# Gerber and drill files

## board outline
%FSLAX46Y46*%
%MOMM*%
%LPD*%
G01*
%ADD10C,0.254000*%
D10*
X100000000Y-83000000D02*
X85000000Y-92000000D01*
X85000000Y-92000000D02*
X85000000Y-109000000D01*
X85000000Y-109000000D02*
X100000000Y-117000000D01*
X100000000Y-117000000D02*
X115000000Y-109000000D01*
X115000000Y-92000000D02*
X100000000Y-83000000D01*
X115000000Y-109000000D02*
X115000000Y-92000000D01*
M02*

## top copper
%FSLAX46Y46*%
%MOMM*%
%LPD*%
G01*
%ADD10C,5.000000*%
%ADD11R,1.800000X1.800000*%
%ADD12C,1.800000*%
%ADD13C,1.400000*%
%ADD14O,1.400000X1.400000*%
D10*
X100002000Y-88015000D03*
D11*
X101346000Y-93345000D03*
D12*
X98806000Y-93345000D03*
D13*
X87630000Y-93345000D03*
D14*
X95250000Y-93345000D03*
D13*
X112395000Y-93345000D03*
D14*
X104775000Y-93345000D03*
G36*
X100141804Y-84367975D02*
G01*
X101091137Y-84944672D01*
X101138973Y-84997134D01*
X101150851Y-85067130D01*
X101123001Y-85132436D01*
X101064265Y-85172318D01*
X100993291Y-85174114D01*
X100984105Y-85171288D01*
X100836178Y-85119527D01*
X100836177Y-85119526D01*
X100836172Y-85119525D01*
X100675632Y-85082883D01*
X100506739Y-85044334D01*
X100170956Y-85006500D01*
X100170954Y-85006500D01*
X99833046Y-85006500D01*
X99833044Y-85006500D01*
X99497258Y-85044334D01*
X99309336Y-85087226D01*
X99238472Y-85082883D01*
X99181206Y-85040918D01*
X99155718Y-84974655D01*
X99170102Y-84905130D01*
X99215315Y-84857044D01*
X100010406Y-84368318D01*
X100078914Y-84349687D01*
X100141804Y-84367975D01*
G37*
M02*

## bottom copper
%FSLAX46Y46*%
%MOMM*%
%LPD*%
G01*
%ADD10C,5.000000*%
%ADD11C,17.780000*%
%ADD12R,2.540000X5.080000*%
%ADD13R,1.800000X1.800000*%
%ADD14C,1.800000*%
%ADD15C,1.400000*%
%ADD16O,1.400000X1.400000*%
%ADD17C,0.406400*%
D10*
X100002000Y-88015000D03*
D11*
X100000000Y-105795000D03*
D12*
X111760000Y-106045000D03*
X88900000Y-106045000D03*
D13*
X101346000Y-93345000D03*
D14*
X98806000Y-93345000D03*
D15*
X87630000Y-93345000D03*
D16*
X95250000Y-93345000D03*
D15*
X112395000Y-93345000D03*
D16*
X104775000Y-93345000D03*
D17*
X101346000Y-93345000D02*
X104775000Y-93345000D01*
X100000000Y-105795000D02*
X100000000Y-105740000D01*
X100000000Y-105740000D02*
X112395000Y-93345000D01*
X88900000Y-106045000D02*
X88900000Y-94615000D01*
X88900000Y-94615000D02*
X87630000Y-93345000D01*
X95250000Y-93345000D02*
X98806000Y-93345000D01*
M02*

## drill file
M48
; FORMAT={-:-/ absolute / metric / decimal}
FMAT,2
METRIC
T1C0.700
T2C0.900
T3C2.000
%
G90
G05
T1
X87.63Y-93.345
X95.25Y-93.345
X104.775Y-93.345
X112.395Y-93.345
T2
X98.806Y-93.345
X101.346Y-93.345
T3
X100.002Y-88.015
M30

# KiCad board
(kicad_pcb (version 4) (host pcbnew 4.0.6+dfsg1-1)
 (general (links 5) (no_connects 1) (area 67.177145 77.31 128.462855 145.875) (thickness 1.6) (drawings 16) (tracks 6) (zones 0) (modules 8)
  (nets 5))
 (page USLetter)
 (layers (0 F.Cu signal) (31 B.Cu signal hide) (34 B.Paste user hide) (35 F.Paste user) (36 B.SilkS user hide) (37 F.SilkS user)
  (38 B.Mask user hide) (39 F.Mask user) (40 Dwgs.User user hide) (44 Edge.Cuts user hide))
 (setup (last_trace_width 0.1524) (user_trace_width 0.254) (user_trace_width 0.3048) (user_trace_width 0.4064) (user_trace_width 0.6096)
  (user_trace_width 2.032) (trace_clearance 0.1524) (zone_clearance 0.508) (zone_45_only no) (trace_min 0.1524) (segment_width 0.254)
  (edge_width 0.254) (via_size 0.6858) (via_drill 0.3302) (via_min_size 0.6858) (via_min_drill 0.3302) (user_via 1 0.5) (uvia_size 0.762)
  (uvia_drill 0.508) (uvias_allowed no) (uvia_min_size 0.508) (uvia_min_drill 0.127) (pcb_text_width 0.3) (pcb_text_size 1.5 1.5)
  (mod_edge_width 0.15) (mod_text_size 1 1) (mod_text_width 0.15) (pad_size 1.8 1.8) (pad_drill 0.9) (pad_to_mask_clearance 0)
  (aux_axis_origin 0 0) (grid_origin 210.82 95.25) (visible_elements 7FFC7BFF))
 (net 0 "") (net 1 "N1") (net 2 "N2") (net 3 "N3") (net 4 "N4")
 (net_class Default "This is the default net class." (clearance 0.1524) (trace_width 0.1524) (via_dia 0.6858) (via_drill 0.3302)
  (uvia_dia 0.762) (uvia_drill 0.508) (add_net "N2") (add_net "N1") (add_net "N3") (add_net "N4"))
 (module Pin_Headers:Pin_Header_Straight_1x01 (layer F.Cu) (at 99.822 88.265)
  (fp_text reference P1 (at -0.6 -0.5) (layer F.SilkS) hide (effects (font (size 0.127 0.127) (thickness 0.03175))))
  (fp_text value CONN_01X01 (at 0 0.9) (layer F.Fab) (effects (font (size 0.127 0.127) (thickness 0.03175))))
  (pad "" thru_hole circle (at 0.18 -0.25) (size 5 5) (drill 2) (layers *.Cu B.Mask)))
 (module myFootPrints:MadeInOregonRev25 (layer F.Cu) (at 108.585 93.091)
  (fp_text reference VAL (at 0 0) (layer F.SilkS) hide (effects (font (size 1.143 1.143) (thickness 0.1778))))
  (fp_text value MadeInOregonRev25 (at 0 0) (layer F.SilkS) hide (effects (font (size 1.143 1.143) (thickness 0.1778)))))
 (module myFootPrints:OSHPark (layer F.Cu) (at 99.949 99.822)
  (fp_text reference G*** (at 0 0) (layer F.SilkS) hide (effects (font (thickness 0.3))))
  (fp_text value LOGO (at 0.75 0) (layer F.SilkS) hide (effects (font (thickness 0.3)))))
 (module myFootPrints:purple (layer F.Cu) (at 99.949 104.902)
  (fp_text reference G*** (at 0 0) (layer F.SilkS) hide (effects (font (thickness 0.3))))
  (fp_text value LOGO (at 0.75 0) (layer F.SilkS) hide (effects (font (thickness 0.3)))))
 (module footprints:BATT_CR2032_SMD (layer B.Cu) (at 100.33 106.045 180)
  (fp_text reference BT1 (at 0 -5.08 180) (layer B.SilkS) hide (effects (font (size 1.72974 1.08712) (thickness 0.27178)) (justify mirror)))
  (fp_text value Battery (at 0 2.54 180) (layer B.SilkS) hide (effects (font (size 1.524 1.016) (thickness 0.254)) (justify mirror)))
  (pad 2 smd circle (at 0.33 0.25 180) (size 17.78 17.78) (layers B.Cu B.Paste B.Mask) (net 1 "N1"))
  (pad 1 smd rect (at -11.43 0 180) (size 2.54 5.08) (layers B.Cu B.Paste B.Mask) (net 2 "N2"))
  (pad 1 smd rect (at 11.43 0 180) (size 2.54 5.08) (layers B.Cu B.Paste B.Mask) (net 2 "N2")))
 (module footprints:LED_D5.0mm (layer F.Cu) (at 101.346 93.345 180)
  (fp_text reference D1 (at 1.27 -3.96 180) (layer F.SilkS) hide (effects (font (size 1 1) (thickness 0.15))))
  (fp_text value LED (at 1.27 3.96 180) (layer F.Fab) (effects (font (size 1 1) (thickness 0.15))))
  (pad 1 thru_hole rect (at 0 0 180) (size 1.8 1.8) (drill 0.9) (layers *.Cu *.Mask) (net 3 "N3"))
  (pad 2 thru_hole circle (at 2.54 0 180) (size 1.8 1.8) (drill 0.9) (layers *.Cu *.Mask) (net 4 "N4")))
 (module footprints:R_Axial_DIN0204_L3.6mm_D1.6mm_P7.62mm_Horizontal (layer F.Cu) (at 87.63 93.345)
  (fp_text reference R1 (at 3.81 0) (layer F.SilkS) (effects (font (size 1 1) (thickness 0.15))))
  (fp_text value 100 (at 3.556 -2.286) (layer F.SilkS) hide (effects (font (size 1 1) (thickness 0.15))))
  (pad 1 thru_hole circle (at 0 0) (size 1.4 1.4) (drill 0.7) (layers *.Cu *.Mask) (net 2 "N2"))
  (pad 2 thru_hole oval (at 7.62 0) (size 1.4 1.4) (drill 0.7) (layers *.Cu *.Mask) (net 4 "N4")))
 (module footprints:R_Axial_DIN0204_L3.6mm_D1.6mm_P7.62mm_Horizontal (layer F.Cu) (at 112.395 93.345 180)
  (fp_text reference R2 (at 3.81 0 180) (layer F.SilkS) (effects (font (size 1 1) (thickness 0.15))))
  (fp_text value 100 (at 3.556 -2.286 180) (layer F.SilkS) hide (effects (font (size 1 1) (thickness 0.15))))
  (pad 1 thru_hole circle (at 0 0 180) (size 1.4 1.4) (drill 0.7) (layers *.Cu *.Mask) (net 1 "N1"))
  (pad 2 thru_hole oval (at 7.62 0 180) (size 1.4 1.4) (drill 0.7) (layers *.Cu *.Mask) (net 3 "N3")))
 (gr_line (start 100 83) (end 85 92) (angle 90) (layer Edge.Cuts) (width 0.254))
 (gr_line (start 85 92) (end 85 109) (angle 90) (layer Edge.Cuts) (width 0.254))
 (gr_line (start 85 109) (end 100 117) (angle 90) (layer Edge.Cuts) (width 0.254))
 (gr_line (start 100 117) (end 115 109) (angle 90) (layer Edge.Cuts) (width 0.254))
 (gr_line (start 115 92) (end 100 83) (angle 90) (layer Edge.Cuts) (width 0.254))
 (gr_line (start 115 109) (end 115 92) (angle 90) (layer Edge.Cuts) (width 0.254))
 (segment (start 101.346 93.345) (end 104.775 93.345) (width 0.4064) (layer B.Cu) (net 3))
 (segment (start 100 105.795) (end 100 105.74) (width 0.4064) (layer B.Cu) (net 1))
 (segment (start 100 105.74) (end 112.395 93.345) (width 0.4064) (layer B.Cu) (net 1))
 (segment (start 88.9 106.045) (end 88.9 94.615) (width 0.4064) (layer B.Cu) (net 2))
 (segment (start 88.9 94.615) (end 87.63 93.345) (width 0.4064) (layer B.Cu) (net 2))
 (segment (start 95.25 93.345) (end 98.806 93.345) (width 0.4064) (layer B.Cu) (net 4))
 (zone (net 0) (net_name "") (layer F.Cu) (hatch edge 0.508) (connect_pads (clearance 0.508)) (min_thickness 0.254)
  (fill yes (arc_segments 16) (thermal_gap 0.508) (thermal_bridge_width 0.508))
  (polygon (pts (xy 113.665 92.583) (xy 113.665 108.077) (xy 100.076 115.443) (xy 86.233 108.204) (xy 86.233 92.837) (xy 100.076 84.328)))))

